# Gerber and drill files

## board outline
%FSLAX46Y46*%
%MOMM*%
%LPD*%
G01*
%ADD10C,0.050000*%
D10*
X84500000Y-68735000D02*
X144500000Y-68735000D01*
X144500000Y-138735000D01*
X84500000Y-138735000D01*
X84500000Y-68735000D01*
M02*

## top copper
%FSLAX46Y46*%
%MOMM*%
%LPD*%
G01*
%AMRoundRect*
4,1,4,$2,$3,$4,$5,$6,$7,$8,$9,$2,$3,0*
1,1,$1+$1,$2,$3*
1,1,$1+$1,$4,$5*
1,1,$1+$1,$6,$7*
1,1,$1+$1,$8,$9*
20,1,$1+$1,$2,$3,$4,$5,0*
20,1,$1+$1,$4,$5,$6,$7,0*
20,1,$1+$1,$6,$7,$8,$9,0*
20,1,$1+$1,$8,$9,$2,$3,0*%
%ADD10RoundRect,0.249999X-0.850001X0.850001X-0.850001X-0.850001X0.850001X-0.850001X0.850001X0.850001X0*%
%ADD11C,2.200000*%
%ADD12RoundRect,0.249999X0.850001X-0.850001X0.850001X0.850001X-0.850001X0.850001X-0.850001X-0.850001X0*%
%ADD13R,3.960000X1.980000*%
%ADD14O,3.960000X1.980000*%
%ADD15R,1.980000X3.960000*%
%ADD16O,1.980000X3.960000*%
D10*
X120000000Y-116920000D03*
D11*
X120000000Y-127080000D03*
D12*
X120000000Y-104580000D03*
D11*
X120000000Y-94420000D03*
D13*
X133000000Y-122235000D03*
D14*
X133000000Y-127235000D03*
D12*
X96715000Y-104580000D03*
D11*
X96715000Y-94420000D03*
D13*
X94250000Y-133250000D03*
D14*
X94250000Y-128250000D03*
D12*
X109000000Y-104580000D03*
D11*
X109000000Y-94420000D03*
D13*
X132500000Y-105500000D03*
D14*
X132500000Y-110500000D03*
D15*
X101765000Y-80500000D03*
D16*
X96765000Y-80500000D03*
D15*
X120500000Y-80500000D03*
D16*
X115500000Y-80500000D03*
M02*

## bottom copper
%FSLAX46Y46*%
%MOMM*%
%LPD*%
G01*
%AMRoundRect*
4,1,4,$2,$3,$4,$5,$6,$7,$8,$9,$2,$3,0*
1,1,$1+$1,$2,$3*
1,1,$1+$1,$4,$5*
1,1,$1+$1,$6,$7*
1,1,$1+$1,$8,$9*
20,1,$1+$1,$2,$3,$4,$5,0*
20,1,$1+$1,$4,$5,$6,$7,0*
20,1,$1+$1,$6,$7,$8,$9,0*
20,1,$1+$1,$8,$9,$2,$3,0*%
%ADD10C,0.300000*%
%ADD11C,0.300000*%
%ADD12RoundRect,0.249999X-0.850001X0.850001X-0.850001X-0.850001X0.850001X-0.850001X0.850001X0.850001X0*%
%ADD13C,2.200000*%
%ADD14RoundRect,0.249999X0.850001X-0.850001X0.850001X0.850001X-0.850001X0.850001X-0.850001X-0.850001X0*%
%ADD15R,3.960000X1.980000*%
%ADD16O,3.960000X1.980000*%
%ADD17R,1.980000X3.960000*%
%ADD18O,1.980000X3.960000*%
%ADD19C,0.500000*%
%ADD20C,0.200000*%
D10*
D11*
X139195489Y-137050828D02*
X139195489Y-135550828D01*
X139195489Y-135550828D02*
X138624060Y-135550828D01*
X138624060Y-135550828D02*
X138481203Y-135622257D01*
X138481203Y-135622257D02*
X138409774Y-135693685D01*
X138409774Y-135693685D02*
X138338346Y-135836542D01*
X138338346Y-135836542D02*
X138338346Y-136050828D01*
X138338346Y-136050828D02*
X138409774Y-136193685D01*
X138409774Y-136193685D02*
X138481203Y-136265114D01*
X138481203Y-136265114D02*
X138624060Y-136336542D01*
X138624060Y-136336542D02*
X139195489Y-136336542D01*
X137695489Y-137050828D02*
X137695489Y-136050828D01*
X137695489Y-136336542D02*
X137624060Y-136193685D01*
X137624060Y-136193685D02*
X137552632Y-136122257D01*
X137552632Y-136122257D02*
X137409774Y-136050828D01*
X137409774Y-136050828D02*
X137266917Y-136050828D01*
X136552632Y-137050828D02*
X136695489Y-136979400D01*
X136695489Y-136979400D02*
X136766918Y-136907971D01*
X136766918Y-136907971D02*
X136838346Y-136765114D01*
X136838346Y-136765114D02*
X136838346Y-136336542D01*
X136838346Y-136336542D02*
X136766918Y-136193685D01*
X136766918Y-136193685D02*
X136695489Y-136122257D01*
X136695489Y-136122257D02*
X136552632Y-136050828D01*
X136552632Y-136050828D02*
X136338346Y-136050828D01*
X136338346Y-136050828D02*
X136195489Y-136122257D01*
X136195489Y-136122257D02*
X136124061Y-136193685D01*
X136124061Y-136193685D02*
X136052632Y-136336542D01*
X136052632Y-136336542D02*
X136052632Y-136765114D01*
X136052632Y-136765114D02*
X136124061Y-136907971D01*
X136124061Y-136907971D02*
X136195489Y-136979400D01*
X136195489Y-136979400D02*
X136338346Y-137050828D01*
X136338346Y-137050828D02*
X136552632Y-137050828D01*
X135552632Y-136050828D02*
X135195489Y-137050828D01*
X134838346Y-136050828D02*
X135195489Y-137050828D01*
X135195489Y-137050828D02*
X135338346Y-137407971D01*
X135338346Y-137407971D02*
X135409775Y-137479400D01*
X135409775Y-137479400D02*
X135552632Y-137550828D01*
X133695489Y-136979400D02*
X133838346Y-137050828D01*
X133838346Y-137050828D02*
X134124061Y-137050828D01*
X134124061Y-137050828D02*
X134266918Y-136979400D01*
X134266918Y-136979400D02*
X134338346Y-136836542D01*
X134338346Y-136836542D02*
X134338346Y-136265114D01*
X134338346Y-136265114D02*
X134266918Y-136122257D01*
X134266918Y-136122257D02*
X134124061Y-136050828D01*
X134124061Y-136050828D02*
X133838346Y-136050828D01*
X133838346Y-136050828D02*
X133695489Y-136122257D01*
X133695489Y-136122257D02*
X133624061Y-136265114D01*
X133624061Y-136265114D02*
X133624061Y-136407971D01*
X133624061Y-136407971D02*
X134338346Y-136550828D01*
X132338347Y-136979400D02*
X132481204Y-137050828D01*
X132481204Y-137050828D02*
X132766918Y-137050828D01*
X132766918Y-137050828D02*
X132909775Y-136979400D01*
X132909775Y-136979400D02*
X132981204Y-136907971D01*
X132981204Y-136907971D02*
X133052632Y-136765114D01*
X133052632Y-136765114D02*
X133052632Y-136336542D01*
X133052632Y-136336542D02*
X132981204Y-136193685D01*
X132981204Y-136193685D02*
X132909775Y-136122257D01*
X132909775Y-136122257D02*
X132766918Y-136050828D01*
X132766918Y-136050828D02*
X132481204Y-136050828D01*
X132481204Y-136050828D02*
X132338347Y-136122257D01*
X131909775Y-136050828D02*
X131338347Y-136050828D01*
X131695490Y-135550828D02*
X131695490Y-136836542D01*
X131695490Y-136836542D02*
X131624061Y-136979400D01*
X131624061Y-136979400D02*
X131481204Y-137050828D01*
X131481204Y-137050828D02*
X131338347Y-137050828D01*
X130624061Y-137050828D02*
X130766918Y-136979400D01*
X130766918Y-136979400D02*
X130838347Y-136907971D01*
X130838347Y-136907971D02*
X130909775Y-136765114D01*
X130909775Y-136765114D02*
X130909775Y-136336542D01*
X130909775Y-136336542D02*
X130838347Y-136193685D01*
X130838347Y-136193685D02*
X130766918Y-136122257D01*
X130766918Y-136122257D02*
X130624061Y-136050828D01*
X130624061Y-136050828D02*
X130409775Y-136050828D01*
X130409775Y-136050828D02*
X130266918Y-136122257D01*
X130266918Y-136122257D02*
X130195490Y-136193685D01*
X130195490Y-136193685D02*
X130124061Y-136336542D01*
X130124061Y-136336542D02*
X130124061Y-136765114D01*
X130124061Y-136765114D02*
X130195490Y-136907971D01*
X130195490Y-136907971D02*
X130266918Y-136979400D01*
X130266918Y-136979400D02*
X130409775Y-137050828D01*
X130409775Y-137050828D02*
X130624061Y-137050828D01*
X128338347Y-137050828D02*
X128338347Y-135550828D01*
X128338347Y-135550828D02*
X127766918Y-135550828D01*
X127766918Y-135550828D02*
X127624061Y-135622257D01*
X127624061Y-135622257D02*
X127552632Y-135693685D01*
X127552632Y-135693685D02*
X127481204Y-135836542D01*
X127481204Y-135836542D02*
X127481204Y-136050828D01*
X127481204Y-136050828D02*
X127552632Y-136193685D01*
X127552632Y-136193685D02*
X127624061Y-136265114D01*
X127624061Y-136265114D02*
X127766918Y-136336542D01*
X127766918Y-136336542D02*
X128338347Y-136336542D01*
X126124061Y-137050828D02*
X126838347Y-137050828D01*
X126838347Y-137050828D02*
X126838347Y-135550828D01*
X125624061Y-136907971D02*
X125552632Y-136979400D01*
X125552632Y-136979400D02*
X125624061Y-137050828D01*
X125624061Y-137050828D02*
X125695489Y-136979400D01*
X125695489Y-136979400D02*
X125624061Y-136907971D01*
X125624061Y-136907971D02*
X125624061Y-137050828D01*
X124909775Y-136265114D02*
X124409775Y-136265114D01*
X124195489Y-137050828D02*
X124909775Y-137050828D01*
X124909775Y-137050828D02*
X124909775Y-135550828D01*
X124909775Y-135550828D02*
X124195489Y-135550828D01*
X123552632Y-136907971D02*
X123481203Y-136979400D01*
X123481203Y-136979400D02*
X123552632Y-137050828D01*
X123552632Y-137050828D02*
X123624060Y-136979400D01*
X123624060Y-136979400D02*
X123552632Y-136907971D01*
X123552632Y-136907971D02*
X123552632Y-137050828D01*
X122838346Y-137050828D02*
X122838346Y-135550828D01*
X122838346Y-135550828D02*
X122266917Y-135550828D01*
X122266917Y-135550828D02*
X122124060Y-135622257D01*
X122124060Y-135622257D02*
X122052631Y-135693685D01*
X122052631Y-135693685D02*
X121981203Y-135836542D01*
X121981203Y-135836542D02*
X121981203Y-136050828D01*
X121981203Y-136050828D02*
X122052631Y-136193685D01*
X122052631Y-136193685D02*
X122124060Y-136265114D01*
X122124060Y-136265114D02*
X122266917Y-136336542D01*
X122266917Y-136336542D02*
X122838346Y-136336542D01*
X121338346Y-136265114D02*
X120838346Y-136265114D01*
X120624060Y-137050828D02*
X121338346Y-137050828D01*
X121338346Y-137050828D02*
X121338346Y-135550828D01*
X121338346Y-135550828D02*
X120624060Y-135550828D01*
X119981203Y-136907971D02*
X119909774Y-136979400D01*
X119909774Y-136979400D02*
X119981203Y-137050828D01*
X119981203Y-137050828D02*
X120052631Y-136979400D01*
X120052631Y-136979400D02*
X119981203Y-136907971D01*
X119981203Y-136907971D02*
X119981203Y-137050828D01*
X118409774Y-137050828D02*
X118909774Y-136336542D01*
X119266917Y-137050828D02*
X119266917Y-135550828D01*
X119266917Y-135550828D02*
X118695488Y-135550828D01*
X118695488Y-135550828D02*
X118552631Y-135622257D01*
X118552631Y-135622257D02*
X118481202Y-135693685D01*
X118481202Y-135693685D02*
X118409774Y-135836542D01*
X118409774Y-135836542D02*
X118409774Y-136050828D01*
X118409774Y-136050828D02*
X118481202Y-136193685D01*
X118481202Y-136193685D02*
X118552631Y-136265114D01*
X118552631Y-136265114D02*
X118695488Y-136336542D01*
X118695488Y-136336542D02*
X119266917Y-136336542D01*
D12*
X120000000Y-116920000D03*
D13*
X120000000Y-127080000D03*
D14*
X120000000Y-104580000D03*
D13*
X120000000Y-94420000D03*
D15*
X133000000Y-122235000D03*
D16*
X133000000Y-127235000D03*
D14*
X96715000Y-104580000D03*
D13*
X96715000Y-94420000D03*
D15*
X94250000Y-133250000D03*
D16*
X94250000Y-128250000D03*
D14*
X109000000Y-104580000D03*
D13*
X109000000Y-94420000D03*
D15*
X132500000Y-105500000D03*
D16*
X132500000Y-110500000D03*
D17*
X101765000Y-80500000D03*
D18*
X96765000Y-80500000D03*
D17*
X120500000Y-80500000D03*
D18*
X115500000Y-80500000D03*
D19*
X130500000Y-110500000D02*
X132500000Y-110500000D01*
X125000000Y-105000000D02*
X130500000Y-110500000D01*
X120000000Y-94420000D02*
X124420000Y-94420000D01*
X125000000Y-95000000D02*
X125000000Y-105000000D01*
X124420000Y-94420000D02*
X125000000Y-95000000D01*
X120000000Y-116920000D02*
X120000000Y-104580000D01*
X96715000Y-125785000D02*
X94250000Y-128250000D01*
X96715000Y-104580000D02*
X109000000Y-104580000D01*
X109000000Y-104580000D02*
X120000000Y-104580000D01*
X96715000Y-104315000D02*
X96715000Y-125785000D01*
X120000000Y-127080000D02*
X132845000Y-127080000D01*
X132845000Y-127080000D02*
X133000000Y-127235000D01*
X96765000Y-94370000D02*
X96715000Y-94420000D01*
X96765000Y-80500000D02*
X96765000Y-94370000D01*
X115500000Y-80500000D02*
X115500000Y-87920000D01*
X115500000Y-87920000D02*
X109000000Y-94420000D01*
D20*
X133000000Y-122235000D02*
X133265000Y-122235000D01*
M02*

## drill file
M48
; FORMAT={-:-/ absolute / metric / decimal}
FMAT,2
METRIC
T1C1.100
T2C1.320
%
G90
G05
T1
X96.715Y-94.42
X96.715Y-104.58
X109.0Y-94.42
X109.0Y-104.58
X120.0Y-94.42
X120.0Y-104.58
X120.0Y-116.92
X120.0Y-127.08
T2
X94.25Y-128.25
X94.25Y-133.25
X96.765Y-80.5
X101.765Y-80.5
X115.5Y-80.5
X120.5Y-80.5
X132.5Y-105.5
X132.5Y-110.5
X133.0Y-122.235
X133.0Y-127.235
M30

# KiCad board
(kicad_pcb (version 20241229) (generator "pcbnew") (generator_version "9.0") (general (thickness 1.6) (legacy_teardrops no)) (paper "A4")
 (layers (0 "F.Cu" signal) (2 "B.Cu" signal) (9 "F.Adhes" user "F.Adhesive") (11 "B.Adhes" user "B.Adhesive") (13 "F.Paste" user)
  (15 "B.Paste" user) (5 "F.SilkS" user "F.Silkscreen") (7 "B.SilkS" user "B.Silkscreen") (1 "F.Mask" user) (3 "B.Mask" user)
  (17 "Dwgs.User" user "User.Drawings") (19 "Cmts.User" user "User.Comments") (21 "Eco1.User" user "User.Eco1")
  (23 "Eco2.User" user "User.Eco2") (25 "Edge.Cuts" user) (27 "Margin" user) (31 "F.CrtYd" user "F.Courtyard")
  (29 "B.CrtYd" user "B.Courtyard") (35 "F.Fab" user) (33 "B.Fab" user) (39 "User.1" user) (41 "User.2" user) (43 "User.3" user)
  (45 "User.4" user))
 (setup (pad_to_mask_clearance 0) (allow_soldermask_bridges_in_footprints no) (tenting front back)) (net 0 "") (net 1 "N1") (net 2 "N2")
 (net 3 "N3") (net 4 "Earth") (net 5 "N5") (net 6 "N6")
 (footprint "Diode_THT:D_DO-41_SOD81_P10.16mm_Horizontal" (layer "F.Cu") (at 120 116.92 -90)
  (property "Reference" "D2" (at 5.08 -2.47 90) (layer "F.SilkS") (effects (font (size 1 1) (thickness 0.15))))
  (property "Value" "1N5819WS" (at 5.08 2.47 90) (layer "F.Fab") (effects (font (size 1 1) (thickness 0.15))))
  (pad "1" thru_hole roundrect (at 0 0 270) (size 2.2 2.2) (drill 1.1) (layers "*.Cu" "*.Mask") (remove_unused_layers no)
   (roundrect_rratio 0.113636) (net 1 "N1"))
  (pad "2" thru_hole circle (at 10.16 0 270) (size 2.2 2.2) (drill 1.1) (layers "*.Cu" "*.Mask") (remove_unused_layers no) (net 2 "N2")))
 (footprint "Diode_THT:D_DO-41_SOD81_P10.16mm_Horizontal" (layer "F.Cu") (at 120 104.58 90)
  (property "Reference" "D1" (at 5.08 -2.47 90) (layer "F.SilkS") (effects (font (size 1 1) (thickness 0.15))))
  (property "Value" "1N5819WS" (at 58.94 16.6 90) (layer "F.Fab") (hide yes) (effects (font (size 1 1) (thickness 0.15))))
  (pad "1" thru_hole roundrect (at 0 0 90) (size 2.2 2.2) (drill 1.1) (layers "*.Cu" "*.Mask") (remove_unused_layers no)
   (roundrect_rratio 0.113636) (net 1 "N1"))
  (pad "2" thru_hole circle (at 10.16 0 90) (size 2.2 2.2) (drill 1.1) (layers "*.Cu" "*.Mask") (remove_unused_layers no) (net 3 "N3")))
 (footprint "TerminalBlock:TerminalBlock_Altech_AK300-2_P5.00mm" (layer "F.Cu") (at 133 122.235 -90)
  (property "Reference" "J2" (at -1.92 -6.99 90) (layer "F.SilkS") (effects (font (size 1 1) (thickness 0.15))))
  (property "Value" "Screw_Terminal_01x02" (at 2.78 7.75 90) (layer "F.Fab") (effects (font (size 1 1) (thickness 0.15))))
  (pad "1" thru_hole rect (at 0 0 270) (size 1.98 3.96) (drill 1.32) (layers "*.Cu" "*.Mask") (remove_unused_layers no) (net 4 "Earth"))
  (pad "2" thru_hole oval (at 5 0 270) (size 1.98 3.96) (drill 1.32) (layers "*.Cu" "*.Mask") (remove_unused_layers no) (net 2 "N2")))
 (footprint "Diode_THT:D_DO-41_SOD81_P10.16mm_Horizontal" (layer "F.Cu") (at 96.715 104.58 90)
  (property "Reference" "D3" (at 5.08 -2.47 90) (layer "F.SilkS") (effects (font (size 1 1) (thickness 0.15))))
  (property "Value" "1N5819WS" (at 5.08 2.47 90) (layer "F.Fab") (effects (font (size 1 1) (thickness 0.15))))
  (pad "1" thru_hole roundrect (at 0 0 90) (size 2.2 2.2) (drill 1.1) (layers "*.Cu" "*.Mask") (remove_unused_layers no)
   (roundrect_rratio 0.113636) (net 1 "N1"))
  (pad "2" thru_hole circle (at 10.16 0 90) (size 2.2 2.2) (drill 1.1) (layers "*.Cu" "*.Mask") (remove_unused_layers no) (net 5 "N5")))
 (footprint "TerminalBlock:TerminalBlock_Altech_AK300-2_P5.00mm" (layer "F.Cu") (at 94.25 133.25 90)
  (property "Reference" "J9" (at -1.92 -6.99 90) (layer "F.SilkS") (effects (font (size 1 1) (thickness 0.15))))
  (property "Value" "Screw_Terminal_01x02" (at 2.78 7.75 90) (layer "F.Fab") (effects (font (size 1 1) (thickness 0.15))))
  (pad "1" thru_hole rect (at 0 0 90) (size 1.98 3.96) (drill 1.32) (layers "*.Cu" "*.Mask") (remove_unused_layers no) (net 4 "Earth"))
  (pad "2" thru_hole oval (at 5 0 90) (size 1.98 3.96) (drill 1.32) (layers "*.Cu" "*.Mask") (remove_unused_layers no) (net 1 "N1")))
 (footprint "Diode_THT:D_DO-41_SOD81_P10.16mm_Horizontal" (layer "F.Cu") (at 109 104.58 90)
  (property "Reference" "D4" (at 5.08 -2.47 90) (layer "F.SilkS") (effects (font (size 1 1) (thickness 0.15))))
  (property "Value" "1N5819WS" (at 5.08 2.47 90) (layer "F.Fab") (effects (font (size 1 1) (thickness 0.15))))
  (pad "1" thru_hole roundrect (at 0 0 90) (size 2.2 2.2) (drill 1.1) (layers "*.Cu" "*.Mask") (remove_unused_layers no)
   (roundrect_rratio 0.113636) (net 1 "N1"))
  (pad "2" thru_hole circle (at 10.16 0 90) (size 2.2 2.2) (drill 1.1) (layers "*.Cu" "*.Mask") (remove_unused_layers no) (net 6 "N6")))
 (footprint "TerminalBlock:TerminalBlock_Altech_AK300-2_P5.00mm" (layer "F.Cu") (at 132.5 105.5 -90)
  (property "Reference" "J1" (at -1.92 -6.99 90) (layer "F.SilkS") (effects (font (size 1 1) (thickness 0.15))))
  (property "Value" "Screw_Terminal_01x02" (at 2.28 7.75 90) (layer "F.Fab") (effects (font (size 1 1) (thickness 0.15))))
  (pad "1" thru_hole rect (at 0 0 270) (size 1.98 3.96) (drill 1.32) (layers "*.Cu" "*.Mask") (remove_unused_layers no) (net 4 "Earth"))
  (pad "2" thru_hole oval (at 5 0 270) (size 1.98 3.96) (drill 1.32) (layers "*.Cu" "*.Mask") (remove_unused_layers no) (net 3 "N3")))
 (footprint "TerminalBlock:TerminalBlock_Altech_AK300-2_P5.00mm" (layer "B.Cu") (at 101.765 80.5 180)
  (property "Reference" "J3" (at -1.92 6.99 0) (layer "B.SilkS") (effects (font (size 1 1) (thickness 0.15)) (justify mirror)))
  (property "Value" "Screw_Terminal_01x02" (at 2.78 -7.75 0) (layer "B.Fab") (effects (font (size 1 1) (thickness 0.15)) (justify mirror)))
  (pad "1" thru_hole rect (at 0 0 180) (size 1.98 3.96) (drill 1.32) (layers "*.Cu" "*.Mask") (remove_unused_layers no) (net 4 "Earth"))
  (pad "2" thru_hole oval (at 5 0 180) (size 1.98 3.96) (drill 1.32) (layers "*.Cu" "*.Mask") (remove_unused_layers no) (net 5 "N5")))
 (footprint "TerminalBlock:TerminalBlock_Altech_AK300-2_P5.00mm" (layer "B.Cu") (at 120.5 80.5 180)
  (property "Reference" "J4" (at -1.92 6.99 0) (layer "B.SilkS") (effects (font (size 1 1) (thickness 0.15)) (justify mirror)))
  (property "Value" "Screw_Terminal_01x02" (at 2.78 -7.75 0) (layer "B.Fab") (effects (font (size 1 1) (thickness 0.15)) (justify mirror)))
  (pad "1" thru_hole rect (at 0 0 180) (size 1.98 3.96) (drill 1.32) (layers "*.Cu" "*.Mask") (remove_unused_layers no) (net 4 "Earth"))
  (pad "2" thru_hole oval (at 5 0 180) (size 1.98 3.96) (drill 1.32) (layers "*.Cu" "*.Mask") (remove_unused_layers no) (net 6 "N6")))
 (gr_rect (start 84.5 68.735) (end 144.5 138.735) (stroke (width 0.05) (type default)) (fill no) (layer "Edge.Cuts"))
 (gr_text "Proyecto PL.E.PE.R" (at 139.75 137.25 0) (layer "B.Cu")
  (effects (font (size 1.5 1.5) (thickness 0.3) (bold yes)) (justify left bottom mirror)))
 (segment (start 130.5 110.5) (end 132.5 110.5) (width 0.5) (layer "B.Cu") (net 3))
 (segment (start 125 105) (end 130.5 110.5) (width 0.5) (layer "B.Cu") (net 3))
 (segment (start 120 94.42) (end 124.42 94.42) (width 0.5) (layer "B.Cu") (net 3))
 (segment (start 125 95) (end 125 105) (width 0.5) (layer "B.Cu") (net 3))
 (segment (start 124.42 94.42) (end 125 95) (width 0.5) (layer "B.Cu") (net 3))
 (segment (start 120 116.92) (end 120 104.58) (width 0.5) (layer "B.Cu") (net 1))
 (segment (start 96.715 125.785) (end 94.25 128.25) (width 0.5) (layer "B.Cu") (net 1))
 (segment (start 96.715 104.58) (end 109 104.58) (width 0.5) (layer "B.Cu") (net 1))
 (segment (start 109 104.58) (end 120 104.58) (width 0.5) (layer "B.Cu") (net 1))
 (segment (start 96.715 104.315) (end 96.715 125.785) (width 0.5) (layer "B.Cu") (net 1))
 (segment (start 120 127.08) (end 132.845 127.08) (width 0.5) (layer "B.Cu") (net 2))
 (segment (start 132.845 127.08) (end 133 127.235) (width 0.5) (layer "B.Cu") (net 2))
 (segment (start 96.765 94.37) (end 96.715 94.42) (width 0.5) (layer "B.Cu") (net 5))
 (segment (start 96.765 80.5) (end 96.765 94.37) (width 0.5) (layer "B.Cu") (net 5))
 (segment (start 115.5 80.5) (end 115.5 87.92) (width 0.5) (layer "B.Cu") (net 6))
 (segment (start 115.5 87.92) (end 109 94.42) (width 0.5) (layer "B.Cu") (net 6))
 (segment (start 133 122.235) (end 133.265 122.235) (width 0.2) (layer "B.Cu") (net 4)))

